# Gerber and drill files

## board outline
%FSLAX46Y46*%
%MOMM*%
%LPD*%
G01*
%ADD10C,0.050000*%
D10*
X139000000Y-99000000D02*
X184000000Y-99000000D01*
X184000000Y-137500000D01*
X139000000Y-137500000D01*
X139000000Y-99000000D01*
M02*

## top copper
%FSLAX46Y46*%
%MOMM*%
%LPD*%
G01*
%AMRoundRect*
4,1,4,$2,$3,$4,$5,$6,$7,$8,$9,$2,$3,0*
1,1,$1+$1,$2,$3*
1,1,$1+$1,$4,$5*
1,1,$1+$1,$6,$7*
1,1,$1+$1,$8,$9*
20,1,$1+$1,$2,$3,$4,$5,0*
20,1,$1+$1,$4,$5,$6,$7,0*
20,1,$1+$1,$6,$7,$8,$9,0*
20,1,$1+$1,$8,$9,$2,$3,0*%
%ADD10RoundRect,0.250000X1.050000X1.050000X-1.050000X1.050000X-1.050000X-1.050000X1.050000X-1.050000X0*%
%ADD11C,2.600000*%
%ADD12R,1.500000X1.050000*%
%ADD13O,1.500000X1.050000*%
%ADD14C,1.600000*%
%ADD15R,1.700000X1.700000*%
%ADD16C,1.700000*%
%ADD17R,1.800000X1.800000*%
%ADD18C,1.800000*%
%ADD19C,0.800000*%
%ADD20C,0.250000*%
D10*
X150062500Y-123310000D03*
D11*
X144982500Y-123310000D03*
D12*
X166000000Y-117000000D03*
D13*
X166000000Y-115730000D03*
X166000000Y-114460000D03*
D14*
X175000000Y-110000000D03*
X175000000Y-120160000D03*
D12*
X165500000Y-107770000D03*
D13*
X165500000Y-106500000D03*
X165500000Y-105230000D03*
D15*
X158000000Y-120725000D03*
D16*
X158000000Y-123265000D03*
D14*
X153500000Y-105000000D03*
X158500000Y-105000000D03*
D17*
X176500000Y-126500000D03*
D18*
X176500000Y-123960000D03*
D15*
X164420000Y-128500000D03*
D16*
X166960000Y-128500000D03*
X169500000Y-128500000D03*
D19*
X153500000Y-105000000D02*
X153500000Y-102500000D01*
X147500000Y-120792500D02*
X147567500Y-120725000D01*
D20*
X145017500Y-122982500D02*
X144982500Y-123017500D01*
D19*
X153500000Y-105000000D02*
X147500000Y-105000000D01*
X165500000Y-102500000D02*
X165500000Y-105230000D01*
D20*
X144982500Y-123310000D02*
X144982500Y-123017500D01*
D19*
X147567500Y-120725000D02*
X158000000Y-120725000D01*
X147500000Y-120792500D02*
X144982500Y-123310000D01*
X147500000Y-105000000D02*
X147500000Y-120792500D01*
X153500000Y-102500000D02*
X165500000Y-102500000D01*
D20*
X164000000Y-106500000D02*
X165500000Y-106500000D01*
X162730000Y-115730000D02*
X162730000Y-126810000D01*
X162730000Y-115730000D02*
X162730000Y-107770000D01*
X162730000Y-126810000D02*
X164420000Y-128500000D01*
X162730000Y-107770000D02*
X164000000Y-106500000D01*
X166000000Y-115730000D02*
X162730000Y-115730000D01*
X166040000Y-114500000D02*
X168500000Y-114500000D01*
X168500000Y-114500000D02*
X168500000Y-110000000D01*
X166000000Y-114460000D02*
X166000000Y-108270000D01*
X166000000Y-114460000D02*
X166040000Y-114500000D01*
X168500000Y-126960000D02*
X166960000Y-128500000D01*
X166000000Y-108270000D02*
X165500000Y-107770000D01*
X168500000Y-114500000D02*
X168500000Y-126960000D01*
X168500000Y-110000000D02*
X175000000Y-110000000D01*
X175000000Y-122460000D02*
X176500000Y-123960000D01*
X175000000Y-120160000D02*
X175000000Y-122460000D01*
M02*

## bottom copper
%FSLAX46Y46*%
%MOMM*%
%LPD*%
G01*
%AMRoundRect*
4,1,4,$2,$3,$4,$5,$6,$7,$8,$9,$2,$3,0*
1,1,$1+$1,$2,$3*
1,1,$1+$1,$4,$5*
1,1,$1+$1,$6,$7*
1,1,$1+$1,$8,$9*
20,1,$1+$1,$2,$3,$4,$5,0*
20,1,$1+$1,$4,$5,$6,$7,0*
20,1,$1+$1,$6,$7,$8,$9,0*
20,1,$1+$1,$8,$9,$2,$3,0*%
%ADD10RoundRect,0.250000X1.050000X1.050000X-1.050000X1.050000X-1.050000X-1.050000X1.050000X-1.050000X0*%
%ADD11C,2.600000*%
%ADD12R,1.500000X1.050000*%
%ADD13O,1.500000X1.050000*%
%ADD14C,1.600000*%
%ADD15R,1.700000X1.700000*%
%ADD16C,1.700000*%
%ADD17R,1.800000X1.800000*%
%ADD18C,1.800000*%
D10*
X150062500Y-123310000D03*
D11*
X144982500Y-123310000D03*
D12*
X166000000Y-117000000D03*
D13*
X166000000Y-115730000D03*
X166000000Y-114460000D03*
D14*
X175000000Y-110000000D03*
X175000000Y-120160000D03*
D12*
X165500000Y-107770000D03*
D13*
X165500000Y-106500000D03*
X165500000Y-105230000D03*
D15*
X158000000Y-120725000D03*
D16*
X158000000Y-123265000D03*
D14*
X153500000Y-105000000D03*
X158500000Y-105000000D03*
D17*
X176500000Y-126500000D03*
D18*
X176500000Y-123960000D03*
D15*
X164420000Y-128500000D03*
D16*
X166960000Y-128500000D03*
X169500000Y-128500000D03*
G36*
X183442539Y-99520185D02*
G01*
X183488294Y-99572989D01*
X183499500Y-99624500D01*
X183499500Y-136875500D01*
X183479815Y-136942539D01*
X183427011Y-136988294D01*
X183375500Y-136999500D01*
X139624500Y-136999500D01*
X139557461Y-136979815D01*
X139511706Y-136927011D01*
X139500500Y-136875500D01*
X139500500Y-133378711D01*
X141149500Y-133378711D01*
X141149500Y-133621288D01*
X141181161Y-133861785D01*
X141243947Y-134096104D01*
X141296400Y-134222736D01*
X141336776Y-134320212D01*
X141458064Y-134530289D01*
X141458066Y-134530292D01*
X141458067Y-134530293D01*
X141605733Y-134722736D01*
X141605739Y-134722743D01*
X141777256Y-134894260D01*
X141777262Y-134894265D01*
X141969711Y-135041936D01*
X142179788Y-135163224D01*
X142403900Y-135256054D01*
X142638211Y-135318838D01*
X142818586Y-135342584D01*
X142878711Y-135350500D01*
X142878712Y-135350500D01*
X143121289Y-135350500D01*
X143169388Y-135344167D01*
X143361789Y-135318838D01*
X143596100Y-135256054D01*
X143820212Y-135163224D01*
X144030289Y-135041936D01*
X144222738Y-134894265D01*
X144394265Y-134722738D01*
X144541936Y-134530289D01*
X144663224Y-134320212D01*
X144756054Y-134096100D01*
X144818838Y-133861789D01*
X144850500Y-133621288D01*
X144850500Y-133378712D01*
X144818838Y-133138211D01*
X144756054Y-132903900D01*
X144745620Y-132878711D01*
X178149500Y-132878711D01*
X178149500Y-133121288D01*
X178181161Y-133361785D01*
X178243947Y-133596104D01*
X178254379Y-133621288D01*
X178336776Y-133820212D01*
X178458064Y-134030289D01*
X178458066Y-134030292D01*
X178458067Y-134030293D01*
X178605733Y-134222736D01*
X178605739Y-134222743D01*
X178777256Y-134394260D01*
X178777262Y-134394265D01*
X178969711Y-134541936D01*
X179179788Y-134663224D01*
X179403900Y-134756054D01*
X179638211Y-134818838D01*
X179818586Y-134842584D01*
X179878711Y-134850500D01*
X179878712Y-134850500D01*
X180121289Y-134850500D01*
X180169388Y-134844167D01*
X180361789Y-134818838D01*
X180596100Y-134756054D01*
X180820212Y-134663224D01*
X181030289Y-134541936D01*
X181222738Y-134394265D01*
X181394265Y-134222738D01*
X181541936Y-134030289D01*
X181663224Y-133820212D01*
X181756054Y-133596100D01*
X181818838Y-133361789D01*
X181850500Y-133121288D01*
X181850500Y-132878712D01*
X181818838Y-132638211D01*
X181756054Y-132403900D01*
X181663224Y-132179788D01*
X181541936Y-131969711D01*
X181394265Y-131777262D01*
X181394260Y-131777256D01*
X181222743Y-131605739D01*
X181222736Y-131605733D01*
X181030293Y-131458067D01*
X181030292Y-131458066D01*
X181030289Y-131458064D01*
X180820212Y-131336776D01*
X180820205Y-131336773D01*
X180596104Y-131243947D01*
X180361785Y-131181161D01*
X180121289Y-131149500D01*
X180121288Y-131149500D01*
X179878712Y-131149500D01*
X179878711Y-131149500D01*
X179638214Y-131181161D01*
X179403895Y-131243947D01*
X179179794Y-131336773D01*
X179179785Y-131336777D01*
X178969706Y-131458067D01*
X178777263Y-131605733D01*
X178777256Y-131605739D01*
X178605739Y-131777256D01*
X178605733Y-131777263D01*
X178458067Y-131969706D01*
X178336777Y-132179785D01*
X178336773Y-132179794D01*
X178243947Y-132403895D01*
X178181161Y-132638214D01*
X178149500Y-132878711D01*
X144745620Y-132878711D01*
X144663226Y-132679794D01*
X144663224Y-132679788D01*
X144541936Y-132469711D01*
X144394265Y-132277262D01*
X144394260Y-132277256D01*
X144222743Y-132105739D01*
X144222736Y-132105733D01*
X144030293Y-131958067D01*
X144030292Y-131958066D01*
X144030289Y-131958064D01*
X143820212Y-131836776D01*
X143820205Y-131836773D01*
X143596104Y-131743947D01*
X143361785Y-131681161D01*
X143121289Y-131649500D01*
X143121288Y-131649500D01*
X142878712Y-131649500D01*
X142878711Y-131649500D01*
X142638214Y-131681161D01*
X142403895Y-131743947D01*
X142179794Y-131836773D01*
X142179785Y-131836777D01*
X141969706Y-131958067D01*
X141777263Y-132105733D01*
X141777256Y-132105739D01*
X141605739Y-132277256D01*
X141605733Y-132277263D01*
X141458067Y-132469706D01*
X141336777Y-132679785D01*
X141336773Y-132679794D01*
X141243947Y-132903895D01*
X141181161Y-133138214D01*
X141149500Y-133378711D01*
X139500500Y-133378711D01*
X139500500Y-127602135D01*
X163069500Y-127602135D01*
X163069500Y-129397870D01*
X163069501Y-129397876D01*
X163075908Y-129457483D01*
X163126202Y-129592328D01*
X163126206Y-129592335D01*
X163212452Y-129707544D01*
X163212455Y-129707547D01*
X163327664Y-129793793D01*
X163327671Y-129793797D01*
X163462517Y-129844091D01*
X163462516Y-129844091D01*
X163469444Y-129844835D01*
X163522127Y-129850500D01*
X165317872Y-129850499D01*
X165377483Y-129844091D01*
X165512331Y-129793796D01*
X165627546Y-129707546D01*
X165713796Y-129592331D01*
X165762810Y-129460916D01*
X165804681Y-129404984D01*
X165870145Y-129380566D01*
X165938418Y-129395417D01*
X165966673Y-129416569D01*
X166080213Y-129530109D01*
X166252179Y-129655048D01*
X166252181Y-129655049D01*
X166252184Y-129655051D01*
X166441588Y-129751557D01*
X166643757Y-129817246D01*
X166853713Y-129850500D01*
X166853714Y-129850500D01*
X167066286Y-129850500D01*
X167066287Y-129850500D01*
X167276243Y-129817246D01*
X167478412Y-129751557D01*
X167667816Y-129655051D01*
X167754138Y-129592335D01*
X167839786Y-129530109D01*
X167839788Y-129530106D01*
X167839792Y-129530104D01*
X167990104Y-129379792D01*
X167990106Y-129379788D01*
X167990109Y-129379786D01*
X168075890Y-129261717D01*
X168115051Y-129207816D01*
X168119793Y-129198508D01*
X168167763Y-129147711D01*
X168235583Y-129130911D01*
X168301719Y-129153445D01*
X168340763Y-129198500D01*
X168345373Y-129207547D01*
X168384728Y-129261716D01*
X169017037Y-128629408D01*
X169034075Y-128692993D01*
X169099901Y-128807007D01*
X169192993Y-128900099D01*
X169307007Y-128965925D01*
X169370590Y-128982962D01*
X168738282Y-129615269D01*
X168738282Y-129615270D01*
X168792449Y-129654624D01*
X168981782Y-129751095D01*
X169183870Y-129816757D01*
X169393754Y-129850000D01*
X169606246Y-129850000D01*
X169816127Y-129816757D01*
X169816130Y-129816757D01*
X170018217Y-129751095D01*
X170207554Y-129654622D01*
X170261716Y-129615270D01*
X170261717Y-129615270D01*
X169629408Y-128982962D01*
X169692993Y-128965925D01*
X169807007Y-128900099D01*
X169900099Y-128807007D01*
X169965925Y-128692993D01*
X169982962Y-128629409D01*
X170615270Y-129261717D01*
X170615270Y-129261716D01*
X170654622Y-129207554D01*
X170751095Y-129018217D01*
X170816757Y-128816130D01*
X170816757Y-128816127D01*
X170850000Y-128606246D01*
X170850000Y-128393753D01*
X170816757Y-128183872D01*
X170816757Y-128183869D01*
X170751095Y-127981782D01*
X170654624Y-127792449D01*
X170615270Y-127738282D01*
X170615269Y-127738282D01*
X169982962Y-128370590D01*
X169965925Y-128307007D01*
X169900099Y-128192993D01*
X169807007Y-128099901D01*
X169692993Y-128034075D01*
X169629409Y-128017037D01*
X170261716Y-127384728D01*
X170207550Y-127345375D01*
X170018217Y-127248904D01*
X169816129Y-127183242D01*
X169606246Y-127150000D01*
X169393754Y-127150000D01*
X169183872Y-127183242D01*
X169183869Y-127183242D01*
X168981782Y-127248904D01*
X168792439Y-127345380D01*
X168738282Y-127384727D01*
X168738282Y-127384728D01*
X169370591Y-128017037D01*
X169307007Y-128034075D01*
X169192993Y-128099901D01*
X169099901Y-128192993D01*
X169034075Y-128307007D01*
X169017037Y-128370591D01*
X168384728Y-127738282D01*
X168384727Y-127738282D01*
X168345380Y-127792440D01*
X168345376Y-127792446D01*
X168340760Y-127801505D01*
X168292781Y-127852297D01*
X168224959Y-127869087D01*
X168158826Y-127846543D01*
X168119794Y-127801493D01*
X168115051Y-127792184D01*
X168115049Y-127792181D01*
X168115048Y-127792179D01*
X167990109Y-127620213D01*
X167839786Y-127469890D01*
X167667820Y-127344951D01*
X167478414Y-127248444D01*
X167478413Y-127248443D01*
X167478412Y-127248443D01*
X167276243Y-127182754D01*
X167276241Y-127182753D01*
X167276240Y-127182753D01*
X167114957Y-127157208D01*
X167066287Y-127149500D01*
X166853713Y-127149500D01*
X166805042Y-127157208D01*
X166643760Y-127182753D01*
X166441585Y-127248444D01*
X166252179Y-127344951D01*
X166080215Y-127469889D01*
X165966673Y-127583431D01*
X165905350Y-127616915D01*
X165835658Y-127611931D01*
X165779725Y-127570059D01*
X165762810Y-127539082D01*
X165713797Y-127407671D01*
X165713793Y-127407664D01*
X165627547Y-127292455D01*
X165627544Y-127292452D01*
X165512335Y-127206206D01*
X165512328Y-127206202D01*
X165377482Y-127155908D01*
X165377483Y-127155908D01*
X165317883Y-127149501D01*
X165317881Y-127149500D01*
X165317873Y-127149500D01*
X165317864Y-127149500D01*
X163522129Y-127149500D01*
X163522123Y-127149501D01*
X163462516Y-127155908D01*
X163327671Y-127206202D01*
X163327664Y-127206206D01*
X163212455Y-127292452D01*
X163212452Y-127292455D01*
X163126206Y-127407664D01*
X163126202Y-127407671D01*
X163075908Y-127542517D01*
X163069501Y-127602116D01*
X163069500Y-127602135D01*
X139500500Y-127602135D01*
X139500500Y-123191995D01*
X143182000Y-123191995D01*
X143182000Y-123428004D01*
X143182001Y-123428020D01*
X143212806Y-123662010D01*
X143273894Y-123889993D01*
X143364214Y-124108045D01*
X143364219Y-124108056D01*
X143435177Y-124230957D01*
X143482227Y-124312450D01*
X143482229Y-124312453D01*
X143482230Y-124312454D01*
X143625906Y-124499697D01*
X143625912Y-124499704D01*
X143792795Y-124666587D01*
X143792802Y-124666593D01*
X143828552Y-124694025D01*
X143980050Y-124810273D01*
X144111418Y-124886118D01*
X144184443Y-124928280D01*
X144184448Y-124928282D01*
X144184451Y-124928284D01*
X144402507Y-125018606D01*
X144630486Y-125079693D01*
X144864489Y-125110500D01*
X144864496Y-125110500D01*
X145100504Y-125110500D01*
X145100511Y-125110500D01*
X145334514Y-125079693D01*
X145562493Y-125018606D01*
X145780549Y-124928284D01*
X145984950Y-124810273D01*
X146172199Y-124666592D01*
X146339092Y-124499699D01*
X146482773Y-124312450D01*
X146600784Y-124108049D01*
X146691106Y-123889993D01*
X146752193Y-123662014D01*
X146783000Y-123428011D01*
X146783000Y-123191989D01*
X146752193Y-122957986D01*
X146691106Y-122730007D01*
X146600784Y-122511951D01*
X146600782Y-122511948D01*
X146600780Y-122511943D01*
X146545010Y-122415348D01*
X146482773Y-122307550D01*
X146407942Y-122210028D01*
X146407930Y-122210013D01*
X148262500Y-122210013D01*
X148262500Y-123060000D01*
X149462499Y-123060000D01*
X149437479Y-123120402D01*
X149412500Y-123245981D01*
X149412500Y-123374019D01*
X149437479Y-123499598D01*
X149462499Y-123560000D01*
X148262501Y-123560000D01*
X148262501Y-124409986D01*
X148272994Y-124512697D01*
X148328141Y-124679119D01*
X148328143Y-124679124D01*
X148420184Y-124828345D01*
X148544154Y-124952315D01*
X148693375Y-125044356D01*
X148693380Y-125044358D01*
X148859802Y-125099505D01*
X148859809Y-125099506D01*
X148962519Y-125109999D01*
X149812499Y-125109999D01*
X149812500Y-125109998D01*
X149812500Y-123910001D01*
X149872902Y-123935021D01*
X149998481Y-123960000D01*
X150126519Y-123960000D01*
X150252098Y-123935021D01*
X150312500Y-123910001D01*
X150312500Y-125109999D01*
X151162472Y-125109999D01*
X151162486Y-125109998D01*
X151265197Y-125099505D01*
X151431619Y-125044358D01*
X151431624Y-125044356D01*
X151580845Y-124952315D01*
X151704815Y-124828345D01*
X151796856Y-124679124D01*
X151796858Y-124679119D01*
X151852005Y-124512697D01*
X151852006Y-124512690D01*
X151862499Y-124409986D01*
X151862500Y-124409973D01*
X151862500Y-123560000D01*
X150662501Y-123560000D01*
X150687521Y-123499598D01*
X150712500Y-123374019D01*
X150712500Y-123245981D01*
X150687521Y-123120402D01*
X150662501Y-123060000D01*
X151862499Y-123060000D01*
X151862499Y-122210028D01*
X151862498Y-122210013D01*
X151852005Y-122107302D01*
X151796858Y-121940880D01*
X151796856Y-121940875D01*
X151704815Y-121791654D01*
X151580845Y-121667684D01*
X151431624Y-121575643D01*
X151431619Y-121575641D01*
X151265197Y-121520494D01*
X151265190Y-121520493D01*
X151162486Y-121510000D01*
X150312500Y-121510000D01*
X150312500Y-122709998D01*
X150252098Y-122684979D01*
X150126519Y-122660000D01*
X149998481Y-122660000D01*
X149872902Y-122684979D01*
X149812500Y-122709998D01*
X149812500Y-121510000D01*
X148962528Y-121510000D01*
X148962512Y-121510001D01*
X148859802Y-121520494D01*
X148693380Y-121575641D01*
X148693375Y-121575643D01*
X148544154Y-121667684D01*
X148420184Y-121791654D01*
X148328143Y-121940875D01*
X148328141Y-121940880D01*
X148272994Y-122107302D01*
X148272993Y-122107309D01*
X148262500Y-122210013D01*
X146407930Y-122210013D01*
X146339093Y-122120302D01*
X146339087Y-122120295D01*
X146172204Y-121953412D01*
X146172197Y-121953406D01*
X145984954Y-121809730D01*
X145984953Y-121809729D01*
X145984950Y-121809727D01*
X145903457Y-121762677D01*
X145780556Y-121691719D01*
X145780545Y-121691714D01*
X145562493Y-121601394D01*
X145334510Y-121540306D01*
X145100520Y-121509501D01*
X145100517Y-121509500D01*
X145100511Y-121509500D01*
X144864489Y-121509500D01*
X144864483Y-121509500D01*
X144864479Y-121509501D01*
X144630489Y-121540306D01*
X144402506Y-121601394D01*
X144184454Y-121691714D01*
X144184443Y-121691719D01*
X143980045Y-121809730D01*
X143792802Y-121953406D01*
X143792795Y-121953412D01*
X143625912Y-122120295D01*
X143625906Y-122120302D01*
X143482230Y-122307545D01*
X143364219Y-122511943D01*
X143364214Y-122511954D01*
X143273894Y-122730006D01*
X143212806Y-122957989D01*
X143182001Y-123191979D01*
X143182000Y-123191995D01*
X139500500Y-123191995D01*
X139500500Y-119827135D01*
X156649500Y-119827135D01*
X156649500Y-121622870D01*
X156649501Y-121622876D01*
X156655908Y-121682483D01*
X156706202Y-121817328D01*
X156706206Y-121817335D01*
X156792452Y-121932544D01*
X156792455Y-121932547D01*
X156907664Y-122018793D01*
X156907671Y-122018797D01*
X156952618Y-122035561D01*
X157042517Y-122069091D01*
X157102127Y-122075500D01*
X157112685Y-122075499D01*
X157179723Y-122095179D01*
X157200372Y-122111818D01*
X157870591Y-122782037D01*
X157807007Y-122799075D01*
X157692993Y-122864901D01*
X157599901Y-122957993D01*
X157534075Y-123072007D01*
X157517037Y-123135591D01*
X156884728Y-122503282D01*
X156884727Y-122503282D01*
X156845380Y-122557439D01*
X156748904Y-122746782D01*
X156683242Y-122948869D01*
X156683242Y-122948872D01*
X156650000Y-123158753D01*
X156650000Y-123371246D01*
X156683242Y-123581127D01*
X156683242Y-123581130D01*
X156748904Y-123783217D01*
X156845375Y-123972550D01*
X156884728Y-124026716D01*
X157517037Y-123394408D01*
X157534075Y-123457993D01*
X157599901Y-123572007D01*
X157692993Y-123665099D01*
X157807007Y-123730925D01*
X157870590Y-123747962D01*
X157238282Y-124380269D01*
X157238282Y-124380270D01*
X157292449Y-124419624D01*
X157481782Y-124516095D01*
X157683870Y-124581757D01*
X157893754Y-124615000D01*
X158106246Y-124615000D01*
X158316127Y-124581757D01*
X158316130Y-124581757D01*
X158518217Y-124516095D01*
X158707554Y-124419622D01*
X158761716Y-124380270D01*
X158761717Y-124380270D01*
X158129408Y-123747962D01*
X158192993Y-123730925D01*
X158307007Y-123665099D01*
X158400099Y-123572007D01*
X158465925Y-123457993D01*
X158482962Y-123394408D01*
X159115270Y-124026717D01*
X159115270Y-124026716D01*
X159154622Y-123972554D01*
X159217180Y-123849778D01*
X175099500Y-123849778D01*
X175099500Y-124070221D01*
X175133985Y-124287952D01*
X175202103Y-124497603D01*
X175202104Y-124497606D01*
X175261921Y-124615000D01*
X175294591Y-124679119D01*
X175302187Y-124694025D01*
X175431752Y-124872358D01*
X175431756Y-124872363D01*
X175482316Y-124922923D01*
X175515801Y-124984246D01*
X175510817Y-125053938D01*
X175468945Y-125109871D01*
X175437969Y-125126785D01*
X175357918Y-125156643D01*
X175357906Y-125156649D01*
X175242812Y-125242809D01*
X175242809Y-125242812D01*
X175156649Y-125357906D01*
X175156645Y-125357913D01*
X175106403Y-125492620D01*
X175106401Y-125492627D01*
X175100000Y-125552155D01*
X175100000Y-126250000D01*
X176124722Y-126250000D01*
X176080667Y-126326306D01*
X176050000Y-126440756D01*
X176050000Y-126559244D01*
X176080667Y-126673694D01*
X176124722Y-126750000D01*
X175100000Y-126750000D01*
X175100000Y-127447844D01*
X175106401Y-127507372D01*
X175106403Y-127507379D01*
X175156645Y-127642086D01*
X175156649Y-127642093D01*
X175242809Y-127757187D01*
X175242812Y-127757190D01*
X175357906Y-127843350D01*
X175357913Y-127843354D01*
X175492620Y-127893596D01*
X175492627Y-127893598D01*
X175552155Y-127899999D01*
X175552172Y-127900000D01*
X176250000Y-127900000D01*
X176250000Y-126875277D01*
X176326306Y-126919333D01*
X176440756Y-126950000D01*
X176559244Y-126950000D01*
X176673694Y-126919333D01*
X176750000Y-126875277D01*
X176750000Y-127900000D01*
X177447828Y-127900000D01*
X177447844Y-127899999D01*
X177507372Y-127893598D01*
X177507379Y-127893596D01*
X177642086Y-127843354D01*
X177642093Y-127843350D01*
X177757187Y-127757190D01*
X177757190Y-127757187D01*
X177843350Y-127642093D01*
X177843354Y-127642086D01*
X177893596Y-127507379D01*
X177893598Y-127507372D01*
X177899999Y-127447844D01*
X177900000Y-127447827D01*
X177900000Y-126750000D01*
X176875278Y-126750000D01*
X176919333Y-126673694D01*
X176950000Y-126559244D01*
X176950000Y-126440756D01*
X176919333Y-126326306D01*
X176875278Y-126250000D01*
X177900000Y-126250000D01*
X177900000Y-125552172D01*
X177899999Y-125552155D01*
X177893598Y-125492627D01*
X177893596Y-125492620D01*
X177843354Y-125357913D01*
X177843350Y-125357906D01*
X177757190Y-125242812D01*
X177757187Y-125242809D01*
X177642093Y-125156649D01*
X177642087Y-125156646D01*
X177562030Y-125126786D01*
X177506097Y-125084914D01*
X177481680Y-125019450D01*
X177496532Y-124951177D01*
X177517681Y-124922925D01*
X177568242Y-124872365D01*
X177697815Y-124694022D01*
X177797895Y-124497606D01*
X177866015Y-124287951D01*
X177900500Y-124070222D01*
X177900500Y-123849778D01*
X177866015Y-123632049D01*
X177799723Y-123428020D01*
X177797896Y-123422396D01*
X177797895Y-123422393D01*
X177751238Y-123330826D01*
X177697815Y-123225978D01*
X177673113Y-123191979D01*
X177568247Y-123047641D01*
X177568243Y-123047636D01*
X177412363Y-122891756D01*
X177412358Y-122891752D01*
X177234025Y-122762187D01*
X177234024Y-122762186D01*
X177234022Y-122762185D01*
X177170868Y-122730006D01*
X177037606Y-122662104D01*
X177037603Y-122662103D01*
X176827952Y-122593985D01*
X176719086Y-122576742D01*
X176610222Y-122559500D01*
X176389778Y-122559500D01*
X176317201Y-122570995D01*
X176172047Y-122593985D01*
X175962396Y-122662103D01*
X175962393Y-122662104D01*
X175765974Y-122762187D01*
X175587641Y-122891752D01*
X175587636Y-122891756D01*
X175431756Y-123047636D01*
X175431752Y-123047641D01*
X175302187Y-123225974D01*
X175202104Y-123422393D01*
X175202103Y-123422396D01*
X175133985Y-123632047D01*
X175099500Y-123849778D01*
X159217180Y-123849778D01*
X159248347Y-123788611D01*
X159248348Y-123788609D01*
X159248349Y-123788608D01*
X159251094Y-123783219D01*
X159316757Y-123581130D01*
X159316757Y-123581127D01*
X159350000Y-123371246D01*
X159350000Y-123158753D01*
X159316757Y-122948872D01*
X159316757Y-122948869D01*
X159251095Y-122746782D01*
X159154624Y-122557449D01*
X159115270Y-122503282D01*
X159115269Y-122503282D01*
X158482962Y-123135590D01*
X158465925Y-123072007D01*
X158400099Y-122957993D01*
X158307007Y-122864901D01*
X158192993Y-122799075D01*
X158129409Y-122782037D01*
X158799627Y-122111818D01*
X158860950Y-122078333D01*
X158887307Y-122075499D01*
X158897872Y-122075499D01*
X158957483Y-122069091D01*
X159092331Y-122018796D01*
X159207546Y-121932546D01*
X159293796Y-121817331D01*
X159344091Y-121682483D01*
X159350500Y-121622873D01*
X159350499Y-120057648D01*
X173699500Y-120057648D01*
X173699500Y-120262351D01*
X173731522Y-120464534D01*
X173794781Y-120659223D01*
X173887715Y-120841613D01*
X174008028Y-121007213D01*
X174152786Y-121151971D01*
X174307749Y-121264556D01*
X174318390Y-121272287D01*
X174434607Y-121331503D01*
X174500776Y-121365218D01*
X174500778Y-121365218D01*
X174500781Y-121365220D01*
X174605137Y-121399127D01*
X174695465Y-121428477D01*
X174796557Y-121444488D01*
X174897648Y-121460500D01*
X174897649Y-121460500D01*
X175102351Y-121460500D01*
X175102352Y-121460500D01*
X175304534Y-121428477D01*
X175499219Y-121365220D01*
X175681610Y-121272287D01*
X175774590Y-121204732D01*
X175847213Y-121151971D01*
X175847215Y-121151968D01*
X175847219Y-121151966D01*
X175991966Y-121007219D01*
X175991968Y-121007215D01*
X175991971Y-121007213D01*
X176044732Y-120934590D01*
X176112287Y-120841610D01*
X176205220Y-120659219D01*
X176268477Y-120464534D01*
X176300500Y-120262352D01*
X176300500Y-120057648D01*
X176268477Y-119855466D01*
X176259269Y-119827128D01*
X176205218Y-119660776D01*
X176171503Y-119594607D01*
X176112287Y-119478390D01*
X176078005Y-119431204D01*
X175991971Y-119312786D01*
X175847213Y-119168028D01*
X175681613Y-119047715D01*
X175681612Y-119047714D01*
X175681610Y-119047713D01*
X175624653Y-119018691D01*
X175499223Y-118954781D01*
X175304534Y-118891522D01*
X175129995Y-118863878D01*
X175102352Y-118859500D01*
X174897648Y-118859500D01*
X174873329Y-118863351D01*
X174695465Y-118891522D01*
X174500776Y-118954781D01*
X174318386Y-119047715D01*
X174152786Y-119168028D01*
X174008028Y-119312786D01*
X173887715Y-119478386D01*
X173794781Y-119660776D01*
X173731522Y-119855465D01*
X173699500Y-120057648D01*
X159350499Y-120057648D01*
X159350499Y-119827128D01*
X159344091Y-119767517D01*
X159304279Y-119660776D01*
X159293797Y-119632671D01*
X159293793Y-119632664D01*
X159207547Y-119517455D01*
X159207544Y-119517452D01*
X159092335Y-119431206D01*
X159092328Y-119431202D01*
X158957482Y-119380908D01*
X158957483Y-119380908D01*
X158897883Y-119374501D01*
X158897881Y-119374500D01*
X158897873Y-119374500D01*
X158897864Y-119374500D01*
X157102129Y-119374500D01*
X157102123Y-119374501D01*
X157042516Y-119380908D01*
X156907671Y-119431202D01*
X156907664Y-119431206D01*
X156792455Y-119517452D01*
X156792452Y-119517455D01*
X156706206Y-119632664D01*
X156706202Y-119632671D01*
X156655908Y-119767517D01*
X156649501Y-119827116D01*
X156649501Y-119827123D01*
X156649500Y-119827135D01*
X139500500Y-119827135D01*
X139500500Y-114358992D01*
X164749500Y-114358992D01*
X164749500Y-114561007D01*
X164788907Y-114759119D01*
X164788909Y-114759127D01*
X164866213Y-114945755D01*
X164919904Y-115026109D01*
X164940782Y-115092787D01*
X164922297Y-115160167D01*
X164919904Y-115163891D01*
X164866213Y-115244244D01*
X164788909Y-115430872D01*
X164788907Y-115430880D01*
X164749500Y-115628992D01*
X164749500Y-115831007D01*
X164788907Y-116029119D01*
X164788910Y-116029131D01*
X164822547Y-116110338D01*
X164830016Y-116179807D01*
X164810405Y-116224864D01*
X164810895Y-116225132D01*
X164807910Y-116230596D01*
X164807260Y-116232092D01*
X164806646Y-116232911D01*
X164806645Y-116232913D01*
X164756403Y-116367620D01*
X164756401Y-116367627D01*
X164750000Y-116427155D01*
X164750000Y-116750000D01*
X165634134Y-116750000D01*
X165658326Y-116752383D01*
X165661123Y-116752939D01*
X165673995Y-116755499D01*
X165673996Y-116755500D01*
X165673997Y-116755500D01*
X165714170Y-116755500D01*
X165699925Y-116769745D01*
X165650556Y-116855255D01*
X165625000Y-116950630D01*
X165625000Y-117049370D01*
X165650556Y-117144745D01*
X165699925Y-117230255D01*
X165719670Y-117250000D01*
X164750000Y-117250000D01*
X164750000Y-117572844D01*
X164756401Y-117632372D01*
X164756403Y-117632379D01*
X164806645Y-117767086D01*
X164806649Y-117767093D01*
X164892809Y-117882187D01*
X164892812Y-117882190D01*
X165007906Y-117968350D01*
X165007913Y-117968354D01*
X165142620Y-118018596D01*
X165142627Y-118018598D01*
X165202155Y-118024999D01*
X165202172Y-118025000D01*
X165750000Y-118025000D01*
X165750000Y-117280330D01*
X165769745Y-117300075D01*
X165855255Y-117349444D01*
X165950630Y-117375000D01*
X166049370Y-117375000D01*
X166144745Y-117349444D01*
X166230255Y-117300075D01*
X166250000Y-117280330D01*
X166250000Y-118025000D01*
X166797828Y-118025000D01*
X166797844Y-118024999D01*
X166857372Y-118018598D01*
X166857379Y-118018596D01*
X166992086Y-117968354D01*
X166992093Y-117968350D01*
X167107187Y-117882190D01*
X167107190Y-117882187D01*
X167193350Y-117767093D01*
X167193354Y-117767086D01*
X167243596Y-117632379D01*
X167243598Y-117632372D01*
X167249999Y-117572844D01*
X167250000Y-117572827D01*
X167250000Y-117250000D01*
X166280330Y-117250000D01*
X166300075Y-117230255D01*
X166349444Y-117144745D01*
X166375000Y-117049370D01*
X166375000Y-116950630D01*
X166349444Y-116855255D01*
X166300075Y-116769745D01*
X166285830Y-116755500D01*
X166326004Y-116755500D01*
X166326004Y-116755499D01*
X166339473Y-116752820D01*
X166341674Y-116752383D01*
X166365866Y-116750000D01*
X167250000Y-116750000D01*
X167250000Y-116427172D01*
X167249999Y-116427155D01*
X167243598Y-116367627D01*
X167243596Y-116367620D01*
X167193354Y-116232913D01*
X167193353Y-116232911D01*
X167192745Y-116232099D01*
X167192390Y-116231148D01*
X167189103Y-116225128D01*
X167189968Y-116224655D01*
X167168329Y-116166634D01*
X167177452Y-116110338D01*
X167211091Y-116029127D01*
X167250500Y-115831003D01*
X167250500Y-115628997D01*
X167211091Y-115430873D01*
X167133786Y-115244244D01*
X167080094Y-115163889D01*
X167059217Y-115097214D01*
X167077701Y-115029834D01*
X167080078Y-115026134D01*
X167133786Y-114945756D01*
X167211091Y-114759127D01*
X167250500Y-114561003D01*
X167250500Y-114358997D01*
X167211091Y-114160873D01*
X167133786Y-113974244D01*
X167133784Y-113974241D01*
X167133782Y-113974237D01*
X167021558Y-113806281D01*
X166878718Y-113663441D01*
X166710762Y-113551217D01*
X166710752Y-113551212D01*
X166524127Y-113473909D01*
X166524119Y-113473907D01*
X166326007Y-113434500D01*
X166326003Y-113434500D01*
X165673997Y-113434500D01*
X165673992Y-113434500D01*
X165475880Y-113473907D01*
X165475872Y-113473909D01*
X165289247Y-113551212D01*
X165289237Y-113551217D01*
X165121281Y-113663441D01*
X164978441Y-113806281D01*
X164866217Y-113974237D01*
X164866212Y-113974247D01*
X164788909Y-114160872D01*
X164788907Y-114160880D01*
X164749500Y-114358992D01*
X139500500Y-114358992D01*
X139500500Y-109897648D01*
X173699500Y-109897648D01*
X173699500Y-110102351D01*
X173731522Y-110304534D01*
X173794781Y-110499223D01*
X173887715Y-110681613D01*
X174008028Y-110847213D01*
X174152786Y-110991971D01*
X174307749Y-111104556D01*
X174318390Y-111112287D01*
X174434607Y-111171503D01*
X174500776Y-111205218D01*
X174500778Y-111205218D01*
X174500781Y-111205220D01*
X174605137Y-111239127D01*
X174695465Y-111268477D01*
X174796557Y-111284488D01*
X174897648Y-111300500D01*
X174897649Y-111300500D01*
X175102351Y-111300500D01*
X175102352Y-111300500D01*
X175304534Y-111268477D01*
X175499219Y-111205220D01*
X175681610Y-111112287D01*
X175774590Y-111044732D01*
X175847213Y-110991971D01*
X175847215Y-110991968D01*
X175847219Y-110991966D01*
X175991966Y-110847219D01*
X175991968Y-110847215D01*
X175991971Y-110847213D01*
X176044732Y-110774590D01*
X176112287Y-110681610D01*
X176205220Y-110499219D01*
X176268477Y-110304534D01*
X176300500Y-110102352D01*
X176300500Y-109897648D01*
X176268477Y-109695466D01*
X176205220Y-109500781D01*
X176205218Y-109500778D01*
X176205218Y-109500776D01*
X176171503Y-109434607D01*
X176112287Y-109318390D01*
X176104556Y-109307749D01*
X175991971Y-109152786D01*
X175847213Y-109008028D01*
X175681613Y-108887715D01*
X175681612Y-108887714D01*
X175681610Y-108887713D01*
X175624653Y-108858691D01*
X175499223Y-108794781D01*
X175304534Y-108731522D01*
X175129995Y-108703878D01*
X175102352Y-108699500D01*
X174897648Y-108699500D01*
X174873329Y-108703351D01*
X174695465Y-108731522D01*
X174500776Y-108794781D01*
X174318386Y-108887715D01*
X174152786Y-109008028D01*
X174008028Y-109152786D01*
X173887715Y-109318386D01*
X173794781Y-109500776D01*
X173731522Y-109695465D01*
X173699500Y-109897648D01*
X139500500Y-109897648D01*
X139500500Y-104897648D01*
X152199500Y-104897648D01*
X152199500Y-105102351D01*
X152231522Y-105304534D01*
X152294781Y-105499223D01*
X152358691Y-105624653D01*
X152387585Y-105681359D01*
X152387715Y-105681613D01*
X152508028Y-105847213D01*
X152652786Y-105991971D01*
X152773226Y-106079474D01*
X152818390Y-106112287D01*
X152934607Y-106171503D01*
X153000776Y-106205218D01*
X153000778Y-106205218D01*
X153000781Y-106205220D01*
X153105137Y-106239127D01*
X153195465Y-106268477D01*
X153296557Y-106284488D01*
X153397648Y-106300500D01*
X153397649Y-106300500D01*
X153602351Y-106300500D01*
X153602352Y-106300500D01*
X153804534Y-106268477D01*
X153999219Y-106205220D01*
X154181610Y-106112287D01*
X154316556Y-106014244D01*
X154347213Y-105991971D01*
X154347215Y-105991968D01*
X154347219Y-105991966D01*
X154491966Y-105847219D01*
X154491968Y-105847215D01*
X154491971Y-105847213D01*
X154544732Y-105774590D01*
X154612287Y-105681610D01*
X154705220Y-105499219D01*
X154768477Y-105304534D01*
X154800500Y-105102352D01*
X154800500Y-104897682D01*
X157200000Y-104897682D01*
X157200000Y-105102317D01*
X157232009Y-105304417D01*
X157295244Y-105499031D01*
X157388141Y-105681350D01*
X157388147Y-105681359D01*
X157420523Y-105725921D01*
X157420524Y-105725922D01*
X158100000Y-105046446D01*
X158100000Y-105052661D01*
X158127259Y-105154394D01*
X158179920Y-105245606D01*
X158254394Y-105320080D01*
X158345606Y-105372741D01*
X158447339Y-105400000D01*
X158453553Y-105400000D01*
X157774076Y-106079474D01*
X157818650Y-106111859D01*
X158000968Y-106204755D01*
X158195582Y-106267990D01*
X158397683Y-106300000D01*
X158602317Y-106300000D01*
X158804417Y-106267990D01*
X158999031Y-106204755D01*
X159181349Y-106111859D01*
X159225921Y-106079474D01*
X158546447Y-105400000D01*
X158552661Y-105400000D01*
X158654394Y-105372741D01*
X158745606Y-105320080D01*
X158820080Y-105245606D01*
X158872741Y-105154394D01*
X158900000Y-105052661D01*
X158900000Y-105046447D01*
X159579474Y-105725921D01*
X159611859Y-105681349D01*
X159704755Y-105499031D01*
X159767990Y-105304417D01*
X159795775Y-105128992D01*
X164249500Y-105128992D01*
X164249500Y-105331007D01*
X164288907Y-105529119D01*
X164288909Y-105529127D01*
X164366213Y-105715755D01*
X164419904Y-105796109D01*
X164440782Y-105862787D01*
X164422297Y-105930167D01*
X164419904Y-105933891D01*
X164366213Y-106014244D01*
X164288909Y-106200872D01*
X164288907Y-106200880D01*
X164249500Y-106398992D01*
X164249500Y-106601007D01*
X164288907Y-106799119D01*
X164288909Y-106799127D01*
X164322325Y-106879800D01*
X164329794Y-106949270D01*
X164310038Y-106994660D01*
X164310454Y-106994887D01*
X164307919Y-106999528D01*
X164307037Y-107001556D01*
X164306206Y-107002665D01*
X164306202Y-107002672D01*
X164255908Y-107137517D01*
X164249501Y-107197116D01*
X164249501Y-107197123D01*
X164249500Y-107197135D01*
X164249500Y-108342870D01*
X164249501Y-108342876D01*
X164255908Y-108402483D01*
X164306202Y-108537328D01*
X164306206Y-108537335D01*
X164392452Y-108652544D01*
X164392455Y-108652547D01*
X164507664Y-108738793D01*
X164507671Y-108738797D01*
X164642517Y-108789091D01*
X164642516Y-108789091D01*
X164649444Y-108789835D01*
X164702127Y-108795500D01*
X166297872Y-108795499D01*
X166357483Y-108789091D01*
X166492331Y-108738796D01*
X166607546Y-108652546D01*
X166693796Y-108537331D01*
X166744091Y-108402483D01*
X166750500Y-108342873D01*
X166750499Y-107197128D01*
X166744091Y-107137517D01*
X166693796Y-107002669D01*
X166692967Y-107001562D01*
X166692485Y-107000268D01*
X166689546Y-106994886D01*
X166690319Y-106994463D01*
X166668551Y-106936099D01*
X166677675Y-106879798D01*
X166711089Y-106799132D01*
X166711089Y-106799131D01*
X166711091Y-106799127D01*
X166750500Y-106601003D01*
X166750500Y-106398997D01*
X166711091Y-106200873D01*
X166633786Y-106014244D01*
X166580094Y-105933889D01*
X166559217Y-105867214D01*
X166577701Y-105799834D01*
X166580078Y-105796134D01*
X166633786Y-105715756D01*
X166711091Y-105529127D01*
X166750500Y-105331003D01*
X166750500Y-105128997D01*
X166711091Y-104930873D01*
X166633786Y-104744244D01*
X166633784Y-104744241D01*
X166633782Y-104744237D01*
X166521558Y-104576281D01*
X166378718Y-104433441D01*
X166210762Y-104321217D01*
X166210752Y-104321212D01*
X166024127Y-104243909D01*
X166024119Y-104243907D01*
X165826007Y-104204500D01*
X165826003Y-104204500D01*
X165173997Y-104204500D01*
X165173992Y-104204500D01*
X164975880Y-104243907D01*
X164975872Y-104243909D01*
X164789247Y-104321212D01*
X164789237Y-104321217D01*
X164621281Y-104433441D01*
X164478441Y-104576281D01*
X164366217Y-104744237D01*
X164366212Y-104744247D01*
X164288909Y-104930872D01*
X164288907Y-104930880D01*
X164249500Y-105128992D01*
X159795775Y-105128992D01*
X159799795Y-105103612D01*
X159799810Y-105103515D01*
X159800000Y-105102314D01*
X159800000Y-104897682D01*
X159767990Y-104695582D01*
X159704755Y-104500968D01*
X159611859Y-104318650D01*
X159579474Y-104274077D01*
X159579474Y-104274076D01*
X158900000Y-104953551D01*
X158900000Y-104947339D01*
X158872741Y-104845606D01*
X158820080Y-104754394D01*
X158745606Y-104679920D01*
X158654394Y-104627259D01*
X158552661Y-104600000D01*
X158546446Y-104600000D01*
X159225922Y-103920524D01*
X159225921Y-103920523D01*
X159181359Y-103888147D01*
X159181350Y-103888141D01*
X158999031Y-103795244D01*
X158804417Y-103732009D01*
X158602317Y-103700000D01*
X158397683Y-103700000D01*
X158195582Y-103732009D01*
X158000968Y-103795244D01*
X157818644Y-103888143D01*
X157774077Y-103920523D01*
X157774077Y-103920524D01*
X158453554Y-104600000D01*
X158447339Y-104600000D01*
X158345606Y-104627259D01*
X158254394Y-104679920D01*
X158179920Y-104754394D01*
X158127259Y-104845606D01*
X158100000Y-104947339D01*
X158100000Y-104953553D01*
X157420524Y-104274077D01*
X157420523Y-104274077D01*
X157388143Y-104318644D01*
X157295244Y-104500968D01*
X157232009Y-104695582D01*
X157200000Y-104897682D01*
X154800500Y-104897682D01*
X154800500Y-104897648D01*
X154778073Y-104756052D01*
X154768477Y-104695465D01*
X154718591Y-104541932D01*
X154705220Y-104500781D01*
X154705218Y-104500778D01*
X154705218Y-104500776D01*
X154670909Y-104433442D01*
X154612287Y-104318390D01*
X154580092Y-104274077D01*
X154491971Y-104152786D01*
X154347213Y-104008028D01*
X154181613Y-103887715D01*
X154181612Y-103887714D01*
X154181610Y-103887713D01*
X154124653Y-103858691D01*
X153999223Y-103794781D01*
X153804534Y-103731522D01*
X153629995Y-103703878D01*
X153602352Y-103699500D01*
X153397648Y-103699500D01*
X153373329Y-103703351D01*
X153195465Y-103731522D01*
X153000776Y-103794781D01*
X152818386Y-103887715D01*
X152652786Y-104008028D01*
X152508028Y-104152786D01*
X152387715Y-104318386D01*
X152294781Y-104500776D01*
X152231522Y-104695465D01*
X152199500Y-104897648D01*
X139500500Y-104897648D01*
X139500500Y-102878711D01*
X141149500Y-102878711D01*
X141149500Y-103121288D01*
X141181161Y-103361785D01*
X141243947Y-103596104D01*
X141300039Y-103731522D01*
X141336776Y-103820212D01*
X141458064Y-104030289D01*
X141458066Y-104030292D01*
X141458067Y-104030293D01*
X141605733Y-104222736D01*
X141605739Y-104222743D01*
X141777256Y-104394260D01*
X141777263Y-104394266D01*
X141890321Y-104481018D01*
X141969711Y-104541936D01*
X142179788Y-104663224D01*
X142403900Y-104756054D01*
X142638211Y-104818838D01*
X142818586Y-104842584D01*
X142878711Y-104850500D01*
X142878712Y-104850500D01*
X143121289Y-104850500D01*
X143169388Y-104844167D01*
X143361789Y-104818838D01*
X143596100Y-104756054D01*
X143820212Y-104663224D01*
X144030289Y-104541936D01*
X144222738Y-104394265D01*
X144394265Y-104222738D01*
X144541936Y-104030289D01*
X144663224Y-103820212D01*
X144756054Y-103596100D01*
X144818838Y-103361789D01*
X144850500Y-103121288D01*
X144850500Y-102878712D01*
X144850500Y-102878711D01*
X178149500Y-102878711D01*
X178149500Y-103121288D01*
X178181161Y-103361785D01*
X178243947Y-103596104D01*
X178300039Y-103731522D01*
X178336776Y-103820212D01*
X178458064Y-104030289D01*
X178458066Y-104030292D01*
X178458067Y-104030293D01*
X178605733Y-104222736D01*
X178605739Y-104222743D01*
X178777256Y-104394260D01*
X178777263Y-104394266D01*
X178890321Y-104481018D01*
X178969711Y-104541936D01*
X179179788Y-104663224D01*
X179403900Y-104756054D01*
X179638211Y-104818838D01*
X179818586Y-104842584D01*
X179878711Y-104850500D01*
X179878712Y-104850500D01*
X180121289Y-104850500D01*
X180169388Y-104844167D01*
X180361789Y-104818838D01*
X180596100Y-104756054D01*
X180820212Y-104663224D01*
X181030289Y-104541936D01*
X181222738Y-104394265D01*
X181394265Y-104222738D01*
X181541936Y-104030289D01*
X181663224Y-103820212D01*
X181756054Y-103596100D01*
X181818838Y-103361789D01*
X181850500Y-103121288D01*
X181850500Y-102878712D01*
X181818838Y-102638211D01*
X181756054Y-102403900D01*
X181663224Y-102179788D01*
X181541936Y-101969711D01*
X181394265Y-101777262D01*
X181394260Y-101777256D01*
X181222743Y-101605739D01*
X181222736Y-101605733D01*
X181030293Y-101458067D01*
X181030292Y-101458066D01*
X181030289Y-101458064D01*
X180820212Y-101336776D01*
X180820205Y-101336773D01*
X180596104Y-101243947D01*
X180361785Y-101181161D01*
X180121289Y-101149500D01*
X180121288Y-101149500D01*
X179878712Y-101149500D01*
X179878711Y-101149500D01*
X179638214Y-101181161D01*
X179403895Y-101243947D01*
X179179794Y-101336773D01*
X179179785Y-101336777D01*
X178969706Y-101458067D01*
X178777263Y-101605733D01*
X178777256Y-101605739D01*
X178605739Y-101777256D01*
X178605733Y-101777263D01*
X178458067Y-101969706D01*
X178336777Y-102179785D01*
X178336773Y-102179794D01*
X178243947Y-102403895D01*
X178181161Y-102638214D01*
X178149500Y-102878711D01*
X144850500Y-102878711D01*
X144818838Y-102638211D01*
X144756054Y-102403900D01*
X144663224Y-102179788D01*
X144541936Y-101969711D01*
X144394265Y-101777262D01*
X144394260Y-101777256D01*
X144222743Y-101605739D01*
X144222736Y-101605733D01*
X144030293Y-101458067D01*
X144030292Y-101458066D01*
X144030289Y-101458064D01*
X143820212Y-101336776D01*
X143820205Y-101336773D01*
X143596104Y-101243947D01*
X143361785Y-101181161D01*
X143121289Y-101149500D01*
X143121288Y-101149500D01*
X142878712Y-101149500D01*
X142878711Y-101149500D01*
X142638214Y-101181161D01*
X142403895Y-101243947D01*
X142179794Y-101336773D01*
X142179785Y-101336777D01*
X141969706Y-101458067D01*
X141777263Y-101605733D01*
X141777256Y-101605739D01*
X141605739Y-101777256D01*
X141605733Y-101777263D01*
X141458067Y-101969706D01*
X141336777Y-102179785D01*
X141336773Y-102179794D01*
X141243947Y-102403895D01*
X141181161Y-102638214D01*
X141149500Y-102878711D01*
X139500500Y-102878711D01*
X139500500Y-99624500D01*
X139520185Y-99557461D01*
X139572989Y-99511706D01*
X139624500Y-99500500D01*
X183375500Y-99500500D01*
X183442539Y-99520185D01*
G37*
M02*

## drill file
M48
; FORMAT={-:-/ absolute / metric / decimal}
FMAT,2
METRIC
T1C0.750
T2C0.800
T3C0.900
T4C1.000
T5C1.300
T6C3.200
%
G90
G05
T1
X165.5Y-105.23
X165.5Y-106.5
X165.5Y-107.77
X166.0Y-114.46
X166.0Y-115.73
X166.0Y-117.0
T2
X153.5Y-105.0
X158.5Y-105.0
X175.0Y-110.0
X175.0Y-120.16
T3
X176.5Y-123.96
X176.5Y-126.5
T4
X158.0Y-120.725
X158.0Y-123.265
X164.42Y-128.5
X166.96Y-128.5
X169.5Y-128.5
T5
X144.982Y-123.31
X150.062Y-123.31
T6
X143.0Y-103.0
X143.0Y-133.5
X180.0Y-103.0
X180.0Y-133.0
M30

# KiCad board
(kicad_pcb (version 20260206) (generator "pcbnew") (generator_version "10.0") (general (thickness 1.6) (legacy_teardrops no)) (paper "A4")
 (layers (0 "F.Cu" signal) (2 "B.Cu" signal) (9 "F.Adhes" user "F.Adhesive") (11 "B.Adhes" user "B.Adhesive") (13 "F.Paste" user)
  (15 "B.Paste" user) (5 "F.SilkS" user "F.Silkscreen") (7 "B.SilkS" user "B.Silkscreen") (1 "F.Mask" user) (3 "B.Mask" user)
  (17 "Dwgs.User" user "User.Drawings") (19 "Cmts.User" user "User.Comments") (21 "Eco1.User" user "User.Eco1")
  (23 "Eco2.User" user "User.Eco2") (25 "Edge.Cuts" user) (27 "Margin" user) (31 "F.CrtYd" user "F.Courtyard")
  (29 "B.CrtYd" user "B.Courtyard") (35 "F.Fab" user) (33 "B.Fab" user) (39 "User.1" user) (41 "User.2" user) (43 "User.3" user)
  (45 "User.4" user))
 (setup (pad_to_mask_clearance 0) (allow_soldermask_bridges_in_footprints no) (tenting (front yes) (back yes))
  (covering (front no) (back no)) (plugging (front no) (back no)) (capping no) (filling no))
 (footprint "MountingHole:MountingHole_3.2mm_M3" (layer "F.Cu") (at 143 103)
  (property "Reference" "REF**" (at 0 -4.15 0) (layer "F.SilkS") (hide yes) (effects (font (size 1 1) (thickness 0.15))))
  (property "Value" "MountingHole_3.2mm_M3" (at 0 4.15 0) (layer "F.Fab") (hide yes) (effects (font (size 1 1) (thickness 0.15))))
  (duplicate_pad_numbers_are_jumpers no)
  (pad "" np_thru_hole circle (at 0 0) (size 3.2 3.2) (drill 3.2) (layers "*.Cu" "*.Mask")))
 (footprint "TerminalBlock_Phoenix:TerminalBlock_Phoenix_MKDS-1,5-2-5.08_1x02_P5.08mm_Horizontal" (layer "F.Cu") (at 150.0625 123.31 180)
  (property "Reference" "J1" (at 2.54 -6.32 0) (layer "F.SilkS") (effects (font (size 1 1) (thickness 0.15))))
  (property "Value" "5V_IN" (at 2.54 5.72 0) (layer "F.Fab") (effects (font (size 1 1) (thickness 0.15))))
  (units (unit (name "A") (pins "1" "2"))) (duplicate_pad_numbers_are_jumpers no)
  (pad "1" thru_hole roundrect (at 0 0 180) (size 2.6 2.6) (drill 1.3) (layers "*.Cu" "*.Mask") (remove_unused_layers no)
   (roundrect_rratio 0.096154) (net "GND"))
  (pad "2" thru_hole circle (at 5.08 0 180) (size 2.6 2.6) (drill 1.3) (layers "*.Cu" "*.Mask") (remove_unused_layers no) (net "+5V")))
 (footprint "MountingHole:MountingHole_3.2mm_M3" (layer "F.Cu") (at 180 103)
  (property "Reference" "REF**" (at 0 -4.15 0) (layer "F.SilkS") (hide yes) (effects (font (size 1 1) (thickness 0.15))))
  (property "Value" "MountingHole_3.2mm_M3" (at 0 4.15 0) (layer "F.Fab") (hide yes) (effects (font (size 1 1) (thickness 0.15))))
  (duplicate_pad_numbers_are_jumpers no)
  (pad "" np_thru_hole circle (at 0 0) (size 3.2 3.2) (drill 3.2) (layers "*.Cu" "*.Mask")))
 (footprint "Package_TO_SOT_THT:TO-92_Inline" (layer "F.Cu") (at 166 117 90)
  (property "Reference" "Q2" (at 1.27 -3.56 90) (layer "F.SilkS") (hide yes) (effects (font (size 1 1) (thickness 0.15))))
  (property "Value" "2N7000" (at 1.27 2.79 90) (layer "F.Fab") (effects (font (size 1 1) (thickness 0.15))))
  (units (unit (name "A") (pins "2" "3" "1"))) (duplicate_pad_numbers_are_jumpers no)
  (pad "1" thru_hole rect (at 0 0 90) (size 1.05 1.5) (drill 0.75) (layers "*.Cu" "*.Mask") (remove_unused_layers no) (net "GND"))
  (pad "2" thru_hole oval (at 1.27 0 90) (size 1.05 1.5) (drill 0.75) (layers "*.Cu" "*.Mask") (remove_unused_layers no) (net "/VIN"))
  (pad "3" thru_hole oval (at 2.54 0 90) (size 1.05 1.5) (drill 0.75) (layers "*.Cu" "*.Mask") (remove_unused_layers no) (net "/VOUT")))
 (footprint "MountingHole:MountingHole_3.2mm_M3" (layer "F.Cu") (at 143 133.5)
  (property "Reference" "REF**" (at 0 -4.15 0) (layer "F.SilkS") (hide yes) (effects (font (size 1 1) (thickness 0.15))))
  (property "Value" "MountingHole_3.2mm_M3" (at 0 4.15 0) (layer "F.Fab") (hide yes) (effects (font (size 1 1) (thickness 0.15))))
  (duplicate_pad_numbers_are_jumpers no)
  (pad "" np_thru_hole circle (at 0 0) (size 3.2 3.2) (drill 3.2) (layers "*.Cu" "*.Mask")))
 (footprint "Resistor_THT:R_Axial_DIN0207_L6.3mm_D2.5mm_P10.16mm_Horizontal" (layer "F.Cu") (at 175 110 -90)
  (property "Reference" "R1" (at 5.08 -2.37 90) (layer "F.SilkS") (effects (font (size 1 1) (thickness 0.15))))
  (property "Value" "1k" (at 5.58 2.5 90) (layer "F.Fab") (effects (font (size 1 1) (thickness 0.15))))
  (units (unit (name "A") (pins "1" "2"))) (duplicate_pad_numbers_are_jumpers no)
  (pad "1" thru_hole circle (at 0 0 270) (size 1.6 1.6) (drill 0.8) (layers "*.Cu" "*.Mask") (remove_unused_layers no) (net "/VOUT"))
  (pad "2" thru_hole circle (at 10.16 0 270) (size 1.6 1.6) (drill 0.8) (layers "*.Cu" "*.Mask") (remove_unused_layers no)
   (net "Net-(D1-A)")))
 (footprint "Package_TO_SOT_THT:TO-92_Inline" (layer "F.Cu") (at 165.5 107.77 90)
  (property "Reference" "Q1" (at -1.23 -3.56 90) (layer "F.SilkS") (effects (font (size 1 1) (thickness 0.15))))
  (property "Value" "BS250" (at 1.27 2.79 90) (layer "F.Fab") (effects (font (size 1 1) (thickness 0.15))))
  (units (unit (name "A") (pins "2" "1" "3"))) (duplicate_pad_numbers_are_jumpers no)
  (pad "1" thru_hole rect (at 0 0 90) (size 1.05 1.5) (drill 0.75) (layers "*.Cu" "*.Mask") (remove_unused_layers no) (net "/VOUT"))
  (pad "2" thru_hole oval (at 1.27 0 90) (size 1.05 1.5) (drill 0.75) (layers "*.Cu" "*.Mask") (remove_unused_layers no) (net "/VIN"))
  (pad "3" thru_hole oval (at 2.54 0 90) (size 1.05 1.5) (drill 0.75) (layers "*.Cu" "*.Mask") (remove_unused_layers no) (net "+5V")))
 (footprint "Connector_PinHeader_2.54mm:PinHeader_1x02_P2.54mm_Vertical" (layer "F.Cu") (at 158 120.725)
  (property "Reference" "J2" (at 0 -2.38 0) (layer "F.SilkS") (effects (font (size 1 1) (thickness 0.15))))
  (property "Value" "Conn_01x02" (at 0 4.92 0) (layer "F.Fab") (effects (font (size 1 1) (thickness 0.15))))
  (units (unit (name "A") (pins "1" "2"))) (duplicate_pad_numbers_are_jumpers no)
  (pad "1" thru_hole rect (at 0 0) (size 1.7 1.7) (drill 1) (layers "*.Cu" "*.Mask") (remove_unused_layers no) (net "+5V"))
  (pad "2" thru_hole circle (at 0 2.54) (size 1.7 1.7) (drill 1) (layers "*.Cu" "*.Mask") (remove_unused_layers no) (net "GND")))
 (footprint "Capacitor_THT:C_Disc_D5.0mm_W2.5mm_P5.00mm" (layer "F.Cu") (at 153.5 105)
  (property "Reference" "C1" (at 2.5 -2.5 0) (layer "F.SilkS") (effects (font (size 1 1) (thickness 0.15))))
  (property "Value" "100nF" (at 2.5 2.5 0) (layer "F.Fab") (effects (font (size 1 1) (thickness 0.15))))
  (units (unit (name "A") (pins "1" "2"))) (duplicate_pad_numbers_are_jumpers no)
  (pad "1" thru_hole circle (at 0 0) (size 1.6 1.6) (drill 0.8) (layers "*.Cu" "*.Mask") (remove_unused_layers no) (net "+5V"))
  (pad "2" thru_hole circle (at 5 0) (size 1.6 1.6) (drill 0.8) (layers "*.Cu" "*.Mask") (remove_unused_layers no) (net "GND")))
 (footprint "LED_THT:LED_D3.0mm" (layer "F.Cu") (at 176.5 126.5 90)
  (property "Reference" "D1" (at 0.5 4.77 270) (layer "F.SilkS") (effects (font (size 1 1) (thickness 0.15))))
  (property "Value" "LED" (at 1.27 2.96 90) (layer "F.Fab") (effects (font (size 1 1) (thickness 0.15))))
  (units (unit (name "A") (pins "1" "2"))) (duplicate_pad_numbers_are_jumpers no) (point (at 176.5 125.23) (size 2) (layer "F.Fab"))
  (pad "1" thru_hole rect (at 0 0 90) (size 1.8 1.8) (drill 0.9) (layers "*.Cu" "*.Mask") (remove_unused_layers no) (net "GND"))
  (pad "2" thru_hole circle (at 2.54 0 90) (size 1.8 1.8) (drill 0.9) (layers "*.Cu" "*.Mask") (remove_unused_layers no) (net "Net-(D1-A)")))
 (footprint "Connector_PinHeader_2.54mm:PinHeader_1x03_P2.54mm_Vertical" (layer "F.Cu") (at 164.42 128.5 90)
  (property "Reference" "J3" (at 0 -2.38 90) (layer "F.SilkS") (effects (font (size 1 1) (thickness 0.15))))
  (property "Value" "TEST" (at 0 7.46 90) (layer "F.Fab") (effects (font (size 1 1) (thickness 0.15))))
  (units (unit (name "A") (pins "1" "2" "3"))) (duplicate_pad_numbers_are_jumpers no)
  (pad "1" thru_hole rect (at 0 0 90) (size 1.7 1.7) (drill 1) (layers "*.Cu" "*.Mask") (remove_unused_layers no) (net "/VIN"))
  (pad "2" thru_hole circle (at 0 2.54 90) (size 1.7 1.7) (drill 1) (layers "*.Cu" "*.Mask") (remove_unused_layers no) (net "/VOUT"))
  (pad "3" thru_hole circle (at 0 5.08 90) (size 1.7 1.7) (drill 1) (layers "*.Cu" "*.Mask") (remove_unused_layers no) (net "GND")))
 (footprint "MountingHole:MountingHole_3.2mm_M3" (layer "F.Cu") (at 180 133)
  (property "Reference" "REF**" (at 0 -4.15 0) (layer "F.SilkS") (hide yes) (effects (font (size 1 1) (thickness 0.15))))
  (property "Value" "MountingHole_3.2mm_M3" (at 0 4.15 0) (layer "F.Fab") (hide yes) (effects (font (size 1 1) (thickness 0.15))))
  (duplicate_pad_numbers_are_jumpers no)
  (pad "" np_thru_hole circle (at 0 0) (size 3.2 3.2) (drill 3.2) (layers "*.Cu" "*.Mask")))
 (gr_rect (start 139 99) (end 184 137.5) (stroke (width 0.05) (type default)) (fill no) (layer "Edge.Cuts"))
 (segment (start 153.5 105) (end 153.5 102.5) (width 0.8) (layer "F.Cu") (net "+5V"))
 (segment (start 147.5 120.7925) (end 147.5675 120.725) (width 0.8) (layer "F.Cu") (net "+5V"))
 (segment (start 145.0175 122.9825) (end 144.9825 123.0175) (width 0.25) (layer "F.Cu") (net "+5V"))
 (segment (start 153.5 105) (end 147.5 105) (width 0.8) (layer "F.Cu") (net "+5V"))
 (segment (start 165.5 102.5) (end 165.5 105.23) (width 0.8) (layer "F.Cu") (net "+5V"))
 (segment (start 144.9825 123.31) (end 144.9825 123.0175) (width 0.25) (layer "F.Cu") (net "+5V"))
 (segment (start 147.5675 120.725) (end 158 120.725) (width 0.8) (layer "F.Cu") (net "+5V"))
 (segment (start 147.5 120.7925) (end 144.9825 123.31) (width 0.8) (layer "F.Cu") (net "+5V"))
 (segment (start 147.5 105) (end 147.5 120.7925) (width 0.8) (layer "F.Cu") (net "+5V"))
 (segment (start 153.5 102.5) (end 165.5 102.5) (width 0.8) (layer "F.Cu") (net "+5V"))
 (segment (start 164 106.5) (end 165.5 106.5) (width 0.25) (layer "F.Cu") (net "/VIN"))
 (segment (start 162.73 115.73) (end 162.73 126.81) (width 0.25) (layer "F.Cu") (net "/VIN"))
 (segment (start 162.73 115.73) (end 162.73 107.77) (width 0.25) (layer "F.Cu") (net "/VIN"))
 (segment (start 162.73 126.81) (end 164.42 128.5) (width 0.25) (layer "F.Cu") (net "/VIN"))
 (segment (start 162.73 107.77) (end 164 106.5) (width 0.25) (layer "F.Cu") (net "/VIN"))
 (segment (start 166 115.73) (end 162.73 115.73) (width 0.25) (layer "F.Cu") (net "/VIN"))
 (segment (start 166.04 114.5) (end 168.5 114.5) (width 0.25) (layer "F.Cu") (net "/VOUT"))
 (segment (start 168.5 114.5) (end 168.5 110) (width 0.25) (layer "F.Cu") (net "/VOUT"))
 (segment (start 166 114.46) (end 166 108.27) (width 0.25) (layer "F.Cu") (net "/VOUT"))
 (segment (start 166 114.46) (end 166.04 114.5) (width 0.25) (layer "F.Cu") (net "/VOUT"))
 (segment (start 168.5 126.96) (end 166.96 128.5) (width 0.25) (layer "F.Cu") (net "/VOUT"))
 (segment (start 166 108.27) (end 165.5 107.77) (width 0.25) (layer "F.Cu") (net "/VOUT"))
 (segment (start 168.5 114.5) (end 168.5 126.96) (width 0.25) (layer "F.Cu") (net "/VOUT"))
 (segment (start 168.5 110) (end 175 110) (width 0.25) (layer "F.Cu") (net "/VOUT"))
 (segment (start 175 122.46) (end 176.5 123.96) (width 0.25) (layer "F.Cu") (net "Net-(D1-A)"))
 (segment (start 175 120.16) (end 175 122.46) (width 0.25) (layer "F.Cu") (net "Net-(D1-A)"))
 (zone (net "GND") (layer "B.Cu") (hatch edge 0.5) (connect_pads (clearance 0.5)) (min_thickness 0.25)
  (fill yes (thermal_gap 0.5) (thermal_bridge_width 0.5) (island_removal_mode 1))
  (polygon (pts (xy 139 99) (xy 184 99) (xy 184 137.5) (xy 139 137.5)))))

